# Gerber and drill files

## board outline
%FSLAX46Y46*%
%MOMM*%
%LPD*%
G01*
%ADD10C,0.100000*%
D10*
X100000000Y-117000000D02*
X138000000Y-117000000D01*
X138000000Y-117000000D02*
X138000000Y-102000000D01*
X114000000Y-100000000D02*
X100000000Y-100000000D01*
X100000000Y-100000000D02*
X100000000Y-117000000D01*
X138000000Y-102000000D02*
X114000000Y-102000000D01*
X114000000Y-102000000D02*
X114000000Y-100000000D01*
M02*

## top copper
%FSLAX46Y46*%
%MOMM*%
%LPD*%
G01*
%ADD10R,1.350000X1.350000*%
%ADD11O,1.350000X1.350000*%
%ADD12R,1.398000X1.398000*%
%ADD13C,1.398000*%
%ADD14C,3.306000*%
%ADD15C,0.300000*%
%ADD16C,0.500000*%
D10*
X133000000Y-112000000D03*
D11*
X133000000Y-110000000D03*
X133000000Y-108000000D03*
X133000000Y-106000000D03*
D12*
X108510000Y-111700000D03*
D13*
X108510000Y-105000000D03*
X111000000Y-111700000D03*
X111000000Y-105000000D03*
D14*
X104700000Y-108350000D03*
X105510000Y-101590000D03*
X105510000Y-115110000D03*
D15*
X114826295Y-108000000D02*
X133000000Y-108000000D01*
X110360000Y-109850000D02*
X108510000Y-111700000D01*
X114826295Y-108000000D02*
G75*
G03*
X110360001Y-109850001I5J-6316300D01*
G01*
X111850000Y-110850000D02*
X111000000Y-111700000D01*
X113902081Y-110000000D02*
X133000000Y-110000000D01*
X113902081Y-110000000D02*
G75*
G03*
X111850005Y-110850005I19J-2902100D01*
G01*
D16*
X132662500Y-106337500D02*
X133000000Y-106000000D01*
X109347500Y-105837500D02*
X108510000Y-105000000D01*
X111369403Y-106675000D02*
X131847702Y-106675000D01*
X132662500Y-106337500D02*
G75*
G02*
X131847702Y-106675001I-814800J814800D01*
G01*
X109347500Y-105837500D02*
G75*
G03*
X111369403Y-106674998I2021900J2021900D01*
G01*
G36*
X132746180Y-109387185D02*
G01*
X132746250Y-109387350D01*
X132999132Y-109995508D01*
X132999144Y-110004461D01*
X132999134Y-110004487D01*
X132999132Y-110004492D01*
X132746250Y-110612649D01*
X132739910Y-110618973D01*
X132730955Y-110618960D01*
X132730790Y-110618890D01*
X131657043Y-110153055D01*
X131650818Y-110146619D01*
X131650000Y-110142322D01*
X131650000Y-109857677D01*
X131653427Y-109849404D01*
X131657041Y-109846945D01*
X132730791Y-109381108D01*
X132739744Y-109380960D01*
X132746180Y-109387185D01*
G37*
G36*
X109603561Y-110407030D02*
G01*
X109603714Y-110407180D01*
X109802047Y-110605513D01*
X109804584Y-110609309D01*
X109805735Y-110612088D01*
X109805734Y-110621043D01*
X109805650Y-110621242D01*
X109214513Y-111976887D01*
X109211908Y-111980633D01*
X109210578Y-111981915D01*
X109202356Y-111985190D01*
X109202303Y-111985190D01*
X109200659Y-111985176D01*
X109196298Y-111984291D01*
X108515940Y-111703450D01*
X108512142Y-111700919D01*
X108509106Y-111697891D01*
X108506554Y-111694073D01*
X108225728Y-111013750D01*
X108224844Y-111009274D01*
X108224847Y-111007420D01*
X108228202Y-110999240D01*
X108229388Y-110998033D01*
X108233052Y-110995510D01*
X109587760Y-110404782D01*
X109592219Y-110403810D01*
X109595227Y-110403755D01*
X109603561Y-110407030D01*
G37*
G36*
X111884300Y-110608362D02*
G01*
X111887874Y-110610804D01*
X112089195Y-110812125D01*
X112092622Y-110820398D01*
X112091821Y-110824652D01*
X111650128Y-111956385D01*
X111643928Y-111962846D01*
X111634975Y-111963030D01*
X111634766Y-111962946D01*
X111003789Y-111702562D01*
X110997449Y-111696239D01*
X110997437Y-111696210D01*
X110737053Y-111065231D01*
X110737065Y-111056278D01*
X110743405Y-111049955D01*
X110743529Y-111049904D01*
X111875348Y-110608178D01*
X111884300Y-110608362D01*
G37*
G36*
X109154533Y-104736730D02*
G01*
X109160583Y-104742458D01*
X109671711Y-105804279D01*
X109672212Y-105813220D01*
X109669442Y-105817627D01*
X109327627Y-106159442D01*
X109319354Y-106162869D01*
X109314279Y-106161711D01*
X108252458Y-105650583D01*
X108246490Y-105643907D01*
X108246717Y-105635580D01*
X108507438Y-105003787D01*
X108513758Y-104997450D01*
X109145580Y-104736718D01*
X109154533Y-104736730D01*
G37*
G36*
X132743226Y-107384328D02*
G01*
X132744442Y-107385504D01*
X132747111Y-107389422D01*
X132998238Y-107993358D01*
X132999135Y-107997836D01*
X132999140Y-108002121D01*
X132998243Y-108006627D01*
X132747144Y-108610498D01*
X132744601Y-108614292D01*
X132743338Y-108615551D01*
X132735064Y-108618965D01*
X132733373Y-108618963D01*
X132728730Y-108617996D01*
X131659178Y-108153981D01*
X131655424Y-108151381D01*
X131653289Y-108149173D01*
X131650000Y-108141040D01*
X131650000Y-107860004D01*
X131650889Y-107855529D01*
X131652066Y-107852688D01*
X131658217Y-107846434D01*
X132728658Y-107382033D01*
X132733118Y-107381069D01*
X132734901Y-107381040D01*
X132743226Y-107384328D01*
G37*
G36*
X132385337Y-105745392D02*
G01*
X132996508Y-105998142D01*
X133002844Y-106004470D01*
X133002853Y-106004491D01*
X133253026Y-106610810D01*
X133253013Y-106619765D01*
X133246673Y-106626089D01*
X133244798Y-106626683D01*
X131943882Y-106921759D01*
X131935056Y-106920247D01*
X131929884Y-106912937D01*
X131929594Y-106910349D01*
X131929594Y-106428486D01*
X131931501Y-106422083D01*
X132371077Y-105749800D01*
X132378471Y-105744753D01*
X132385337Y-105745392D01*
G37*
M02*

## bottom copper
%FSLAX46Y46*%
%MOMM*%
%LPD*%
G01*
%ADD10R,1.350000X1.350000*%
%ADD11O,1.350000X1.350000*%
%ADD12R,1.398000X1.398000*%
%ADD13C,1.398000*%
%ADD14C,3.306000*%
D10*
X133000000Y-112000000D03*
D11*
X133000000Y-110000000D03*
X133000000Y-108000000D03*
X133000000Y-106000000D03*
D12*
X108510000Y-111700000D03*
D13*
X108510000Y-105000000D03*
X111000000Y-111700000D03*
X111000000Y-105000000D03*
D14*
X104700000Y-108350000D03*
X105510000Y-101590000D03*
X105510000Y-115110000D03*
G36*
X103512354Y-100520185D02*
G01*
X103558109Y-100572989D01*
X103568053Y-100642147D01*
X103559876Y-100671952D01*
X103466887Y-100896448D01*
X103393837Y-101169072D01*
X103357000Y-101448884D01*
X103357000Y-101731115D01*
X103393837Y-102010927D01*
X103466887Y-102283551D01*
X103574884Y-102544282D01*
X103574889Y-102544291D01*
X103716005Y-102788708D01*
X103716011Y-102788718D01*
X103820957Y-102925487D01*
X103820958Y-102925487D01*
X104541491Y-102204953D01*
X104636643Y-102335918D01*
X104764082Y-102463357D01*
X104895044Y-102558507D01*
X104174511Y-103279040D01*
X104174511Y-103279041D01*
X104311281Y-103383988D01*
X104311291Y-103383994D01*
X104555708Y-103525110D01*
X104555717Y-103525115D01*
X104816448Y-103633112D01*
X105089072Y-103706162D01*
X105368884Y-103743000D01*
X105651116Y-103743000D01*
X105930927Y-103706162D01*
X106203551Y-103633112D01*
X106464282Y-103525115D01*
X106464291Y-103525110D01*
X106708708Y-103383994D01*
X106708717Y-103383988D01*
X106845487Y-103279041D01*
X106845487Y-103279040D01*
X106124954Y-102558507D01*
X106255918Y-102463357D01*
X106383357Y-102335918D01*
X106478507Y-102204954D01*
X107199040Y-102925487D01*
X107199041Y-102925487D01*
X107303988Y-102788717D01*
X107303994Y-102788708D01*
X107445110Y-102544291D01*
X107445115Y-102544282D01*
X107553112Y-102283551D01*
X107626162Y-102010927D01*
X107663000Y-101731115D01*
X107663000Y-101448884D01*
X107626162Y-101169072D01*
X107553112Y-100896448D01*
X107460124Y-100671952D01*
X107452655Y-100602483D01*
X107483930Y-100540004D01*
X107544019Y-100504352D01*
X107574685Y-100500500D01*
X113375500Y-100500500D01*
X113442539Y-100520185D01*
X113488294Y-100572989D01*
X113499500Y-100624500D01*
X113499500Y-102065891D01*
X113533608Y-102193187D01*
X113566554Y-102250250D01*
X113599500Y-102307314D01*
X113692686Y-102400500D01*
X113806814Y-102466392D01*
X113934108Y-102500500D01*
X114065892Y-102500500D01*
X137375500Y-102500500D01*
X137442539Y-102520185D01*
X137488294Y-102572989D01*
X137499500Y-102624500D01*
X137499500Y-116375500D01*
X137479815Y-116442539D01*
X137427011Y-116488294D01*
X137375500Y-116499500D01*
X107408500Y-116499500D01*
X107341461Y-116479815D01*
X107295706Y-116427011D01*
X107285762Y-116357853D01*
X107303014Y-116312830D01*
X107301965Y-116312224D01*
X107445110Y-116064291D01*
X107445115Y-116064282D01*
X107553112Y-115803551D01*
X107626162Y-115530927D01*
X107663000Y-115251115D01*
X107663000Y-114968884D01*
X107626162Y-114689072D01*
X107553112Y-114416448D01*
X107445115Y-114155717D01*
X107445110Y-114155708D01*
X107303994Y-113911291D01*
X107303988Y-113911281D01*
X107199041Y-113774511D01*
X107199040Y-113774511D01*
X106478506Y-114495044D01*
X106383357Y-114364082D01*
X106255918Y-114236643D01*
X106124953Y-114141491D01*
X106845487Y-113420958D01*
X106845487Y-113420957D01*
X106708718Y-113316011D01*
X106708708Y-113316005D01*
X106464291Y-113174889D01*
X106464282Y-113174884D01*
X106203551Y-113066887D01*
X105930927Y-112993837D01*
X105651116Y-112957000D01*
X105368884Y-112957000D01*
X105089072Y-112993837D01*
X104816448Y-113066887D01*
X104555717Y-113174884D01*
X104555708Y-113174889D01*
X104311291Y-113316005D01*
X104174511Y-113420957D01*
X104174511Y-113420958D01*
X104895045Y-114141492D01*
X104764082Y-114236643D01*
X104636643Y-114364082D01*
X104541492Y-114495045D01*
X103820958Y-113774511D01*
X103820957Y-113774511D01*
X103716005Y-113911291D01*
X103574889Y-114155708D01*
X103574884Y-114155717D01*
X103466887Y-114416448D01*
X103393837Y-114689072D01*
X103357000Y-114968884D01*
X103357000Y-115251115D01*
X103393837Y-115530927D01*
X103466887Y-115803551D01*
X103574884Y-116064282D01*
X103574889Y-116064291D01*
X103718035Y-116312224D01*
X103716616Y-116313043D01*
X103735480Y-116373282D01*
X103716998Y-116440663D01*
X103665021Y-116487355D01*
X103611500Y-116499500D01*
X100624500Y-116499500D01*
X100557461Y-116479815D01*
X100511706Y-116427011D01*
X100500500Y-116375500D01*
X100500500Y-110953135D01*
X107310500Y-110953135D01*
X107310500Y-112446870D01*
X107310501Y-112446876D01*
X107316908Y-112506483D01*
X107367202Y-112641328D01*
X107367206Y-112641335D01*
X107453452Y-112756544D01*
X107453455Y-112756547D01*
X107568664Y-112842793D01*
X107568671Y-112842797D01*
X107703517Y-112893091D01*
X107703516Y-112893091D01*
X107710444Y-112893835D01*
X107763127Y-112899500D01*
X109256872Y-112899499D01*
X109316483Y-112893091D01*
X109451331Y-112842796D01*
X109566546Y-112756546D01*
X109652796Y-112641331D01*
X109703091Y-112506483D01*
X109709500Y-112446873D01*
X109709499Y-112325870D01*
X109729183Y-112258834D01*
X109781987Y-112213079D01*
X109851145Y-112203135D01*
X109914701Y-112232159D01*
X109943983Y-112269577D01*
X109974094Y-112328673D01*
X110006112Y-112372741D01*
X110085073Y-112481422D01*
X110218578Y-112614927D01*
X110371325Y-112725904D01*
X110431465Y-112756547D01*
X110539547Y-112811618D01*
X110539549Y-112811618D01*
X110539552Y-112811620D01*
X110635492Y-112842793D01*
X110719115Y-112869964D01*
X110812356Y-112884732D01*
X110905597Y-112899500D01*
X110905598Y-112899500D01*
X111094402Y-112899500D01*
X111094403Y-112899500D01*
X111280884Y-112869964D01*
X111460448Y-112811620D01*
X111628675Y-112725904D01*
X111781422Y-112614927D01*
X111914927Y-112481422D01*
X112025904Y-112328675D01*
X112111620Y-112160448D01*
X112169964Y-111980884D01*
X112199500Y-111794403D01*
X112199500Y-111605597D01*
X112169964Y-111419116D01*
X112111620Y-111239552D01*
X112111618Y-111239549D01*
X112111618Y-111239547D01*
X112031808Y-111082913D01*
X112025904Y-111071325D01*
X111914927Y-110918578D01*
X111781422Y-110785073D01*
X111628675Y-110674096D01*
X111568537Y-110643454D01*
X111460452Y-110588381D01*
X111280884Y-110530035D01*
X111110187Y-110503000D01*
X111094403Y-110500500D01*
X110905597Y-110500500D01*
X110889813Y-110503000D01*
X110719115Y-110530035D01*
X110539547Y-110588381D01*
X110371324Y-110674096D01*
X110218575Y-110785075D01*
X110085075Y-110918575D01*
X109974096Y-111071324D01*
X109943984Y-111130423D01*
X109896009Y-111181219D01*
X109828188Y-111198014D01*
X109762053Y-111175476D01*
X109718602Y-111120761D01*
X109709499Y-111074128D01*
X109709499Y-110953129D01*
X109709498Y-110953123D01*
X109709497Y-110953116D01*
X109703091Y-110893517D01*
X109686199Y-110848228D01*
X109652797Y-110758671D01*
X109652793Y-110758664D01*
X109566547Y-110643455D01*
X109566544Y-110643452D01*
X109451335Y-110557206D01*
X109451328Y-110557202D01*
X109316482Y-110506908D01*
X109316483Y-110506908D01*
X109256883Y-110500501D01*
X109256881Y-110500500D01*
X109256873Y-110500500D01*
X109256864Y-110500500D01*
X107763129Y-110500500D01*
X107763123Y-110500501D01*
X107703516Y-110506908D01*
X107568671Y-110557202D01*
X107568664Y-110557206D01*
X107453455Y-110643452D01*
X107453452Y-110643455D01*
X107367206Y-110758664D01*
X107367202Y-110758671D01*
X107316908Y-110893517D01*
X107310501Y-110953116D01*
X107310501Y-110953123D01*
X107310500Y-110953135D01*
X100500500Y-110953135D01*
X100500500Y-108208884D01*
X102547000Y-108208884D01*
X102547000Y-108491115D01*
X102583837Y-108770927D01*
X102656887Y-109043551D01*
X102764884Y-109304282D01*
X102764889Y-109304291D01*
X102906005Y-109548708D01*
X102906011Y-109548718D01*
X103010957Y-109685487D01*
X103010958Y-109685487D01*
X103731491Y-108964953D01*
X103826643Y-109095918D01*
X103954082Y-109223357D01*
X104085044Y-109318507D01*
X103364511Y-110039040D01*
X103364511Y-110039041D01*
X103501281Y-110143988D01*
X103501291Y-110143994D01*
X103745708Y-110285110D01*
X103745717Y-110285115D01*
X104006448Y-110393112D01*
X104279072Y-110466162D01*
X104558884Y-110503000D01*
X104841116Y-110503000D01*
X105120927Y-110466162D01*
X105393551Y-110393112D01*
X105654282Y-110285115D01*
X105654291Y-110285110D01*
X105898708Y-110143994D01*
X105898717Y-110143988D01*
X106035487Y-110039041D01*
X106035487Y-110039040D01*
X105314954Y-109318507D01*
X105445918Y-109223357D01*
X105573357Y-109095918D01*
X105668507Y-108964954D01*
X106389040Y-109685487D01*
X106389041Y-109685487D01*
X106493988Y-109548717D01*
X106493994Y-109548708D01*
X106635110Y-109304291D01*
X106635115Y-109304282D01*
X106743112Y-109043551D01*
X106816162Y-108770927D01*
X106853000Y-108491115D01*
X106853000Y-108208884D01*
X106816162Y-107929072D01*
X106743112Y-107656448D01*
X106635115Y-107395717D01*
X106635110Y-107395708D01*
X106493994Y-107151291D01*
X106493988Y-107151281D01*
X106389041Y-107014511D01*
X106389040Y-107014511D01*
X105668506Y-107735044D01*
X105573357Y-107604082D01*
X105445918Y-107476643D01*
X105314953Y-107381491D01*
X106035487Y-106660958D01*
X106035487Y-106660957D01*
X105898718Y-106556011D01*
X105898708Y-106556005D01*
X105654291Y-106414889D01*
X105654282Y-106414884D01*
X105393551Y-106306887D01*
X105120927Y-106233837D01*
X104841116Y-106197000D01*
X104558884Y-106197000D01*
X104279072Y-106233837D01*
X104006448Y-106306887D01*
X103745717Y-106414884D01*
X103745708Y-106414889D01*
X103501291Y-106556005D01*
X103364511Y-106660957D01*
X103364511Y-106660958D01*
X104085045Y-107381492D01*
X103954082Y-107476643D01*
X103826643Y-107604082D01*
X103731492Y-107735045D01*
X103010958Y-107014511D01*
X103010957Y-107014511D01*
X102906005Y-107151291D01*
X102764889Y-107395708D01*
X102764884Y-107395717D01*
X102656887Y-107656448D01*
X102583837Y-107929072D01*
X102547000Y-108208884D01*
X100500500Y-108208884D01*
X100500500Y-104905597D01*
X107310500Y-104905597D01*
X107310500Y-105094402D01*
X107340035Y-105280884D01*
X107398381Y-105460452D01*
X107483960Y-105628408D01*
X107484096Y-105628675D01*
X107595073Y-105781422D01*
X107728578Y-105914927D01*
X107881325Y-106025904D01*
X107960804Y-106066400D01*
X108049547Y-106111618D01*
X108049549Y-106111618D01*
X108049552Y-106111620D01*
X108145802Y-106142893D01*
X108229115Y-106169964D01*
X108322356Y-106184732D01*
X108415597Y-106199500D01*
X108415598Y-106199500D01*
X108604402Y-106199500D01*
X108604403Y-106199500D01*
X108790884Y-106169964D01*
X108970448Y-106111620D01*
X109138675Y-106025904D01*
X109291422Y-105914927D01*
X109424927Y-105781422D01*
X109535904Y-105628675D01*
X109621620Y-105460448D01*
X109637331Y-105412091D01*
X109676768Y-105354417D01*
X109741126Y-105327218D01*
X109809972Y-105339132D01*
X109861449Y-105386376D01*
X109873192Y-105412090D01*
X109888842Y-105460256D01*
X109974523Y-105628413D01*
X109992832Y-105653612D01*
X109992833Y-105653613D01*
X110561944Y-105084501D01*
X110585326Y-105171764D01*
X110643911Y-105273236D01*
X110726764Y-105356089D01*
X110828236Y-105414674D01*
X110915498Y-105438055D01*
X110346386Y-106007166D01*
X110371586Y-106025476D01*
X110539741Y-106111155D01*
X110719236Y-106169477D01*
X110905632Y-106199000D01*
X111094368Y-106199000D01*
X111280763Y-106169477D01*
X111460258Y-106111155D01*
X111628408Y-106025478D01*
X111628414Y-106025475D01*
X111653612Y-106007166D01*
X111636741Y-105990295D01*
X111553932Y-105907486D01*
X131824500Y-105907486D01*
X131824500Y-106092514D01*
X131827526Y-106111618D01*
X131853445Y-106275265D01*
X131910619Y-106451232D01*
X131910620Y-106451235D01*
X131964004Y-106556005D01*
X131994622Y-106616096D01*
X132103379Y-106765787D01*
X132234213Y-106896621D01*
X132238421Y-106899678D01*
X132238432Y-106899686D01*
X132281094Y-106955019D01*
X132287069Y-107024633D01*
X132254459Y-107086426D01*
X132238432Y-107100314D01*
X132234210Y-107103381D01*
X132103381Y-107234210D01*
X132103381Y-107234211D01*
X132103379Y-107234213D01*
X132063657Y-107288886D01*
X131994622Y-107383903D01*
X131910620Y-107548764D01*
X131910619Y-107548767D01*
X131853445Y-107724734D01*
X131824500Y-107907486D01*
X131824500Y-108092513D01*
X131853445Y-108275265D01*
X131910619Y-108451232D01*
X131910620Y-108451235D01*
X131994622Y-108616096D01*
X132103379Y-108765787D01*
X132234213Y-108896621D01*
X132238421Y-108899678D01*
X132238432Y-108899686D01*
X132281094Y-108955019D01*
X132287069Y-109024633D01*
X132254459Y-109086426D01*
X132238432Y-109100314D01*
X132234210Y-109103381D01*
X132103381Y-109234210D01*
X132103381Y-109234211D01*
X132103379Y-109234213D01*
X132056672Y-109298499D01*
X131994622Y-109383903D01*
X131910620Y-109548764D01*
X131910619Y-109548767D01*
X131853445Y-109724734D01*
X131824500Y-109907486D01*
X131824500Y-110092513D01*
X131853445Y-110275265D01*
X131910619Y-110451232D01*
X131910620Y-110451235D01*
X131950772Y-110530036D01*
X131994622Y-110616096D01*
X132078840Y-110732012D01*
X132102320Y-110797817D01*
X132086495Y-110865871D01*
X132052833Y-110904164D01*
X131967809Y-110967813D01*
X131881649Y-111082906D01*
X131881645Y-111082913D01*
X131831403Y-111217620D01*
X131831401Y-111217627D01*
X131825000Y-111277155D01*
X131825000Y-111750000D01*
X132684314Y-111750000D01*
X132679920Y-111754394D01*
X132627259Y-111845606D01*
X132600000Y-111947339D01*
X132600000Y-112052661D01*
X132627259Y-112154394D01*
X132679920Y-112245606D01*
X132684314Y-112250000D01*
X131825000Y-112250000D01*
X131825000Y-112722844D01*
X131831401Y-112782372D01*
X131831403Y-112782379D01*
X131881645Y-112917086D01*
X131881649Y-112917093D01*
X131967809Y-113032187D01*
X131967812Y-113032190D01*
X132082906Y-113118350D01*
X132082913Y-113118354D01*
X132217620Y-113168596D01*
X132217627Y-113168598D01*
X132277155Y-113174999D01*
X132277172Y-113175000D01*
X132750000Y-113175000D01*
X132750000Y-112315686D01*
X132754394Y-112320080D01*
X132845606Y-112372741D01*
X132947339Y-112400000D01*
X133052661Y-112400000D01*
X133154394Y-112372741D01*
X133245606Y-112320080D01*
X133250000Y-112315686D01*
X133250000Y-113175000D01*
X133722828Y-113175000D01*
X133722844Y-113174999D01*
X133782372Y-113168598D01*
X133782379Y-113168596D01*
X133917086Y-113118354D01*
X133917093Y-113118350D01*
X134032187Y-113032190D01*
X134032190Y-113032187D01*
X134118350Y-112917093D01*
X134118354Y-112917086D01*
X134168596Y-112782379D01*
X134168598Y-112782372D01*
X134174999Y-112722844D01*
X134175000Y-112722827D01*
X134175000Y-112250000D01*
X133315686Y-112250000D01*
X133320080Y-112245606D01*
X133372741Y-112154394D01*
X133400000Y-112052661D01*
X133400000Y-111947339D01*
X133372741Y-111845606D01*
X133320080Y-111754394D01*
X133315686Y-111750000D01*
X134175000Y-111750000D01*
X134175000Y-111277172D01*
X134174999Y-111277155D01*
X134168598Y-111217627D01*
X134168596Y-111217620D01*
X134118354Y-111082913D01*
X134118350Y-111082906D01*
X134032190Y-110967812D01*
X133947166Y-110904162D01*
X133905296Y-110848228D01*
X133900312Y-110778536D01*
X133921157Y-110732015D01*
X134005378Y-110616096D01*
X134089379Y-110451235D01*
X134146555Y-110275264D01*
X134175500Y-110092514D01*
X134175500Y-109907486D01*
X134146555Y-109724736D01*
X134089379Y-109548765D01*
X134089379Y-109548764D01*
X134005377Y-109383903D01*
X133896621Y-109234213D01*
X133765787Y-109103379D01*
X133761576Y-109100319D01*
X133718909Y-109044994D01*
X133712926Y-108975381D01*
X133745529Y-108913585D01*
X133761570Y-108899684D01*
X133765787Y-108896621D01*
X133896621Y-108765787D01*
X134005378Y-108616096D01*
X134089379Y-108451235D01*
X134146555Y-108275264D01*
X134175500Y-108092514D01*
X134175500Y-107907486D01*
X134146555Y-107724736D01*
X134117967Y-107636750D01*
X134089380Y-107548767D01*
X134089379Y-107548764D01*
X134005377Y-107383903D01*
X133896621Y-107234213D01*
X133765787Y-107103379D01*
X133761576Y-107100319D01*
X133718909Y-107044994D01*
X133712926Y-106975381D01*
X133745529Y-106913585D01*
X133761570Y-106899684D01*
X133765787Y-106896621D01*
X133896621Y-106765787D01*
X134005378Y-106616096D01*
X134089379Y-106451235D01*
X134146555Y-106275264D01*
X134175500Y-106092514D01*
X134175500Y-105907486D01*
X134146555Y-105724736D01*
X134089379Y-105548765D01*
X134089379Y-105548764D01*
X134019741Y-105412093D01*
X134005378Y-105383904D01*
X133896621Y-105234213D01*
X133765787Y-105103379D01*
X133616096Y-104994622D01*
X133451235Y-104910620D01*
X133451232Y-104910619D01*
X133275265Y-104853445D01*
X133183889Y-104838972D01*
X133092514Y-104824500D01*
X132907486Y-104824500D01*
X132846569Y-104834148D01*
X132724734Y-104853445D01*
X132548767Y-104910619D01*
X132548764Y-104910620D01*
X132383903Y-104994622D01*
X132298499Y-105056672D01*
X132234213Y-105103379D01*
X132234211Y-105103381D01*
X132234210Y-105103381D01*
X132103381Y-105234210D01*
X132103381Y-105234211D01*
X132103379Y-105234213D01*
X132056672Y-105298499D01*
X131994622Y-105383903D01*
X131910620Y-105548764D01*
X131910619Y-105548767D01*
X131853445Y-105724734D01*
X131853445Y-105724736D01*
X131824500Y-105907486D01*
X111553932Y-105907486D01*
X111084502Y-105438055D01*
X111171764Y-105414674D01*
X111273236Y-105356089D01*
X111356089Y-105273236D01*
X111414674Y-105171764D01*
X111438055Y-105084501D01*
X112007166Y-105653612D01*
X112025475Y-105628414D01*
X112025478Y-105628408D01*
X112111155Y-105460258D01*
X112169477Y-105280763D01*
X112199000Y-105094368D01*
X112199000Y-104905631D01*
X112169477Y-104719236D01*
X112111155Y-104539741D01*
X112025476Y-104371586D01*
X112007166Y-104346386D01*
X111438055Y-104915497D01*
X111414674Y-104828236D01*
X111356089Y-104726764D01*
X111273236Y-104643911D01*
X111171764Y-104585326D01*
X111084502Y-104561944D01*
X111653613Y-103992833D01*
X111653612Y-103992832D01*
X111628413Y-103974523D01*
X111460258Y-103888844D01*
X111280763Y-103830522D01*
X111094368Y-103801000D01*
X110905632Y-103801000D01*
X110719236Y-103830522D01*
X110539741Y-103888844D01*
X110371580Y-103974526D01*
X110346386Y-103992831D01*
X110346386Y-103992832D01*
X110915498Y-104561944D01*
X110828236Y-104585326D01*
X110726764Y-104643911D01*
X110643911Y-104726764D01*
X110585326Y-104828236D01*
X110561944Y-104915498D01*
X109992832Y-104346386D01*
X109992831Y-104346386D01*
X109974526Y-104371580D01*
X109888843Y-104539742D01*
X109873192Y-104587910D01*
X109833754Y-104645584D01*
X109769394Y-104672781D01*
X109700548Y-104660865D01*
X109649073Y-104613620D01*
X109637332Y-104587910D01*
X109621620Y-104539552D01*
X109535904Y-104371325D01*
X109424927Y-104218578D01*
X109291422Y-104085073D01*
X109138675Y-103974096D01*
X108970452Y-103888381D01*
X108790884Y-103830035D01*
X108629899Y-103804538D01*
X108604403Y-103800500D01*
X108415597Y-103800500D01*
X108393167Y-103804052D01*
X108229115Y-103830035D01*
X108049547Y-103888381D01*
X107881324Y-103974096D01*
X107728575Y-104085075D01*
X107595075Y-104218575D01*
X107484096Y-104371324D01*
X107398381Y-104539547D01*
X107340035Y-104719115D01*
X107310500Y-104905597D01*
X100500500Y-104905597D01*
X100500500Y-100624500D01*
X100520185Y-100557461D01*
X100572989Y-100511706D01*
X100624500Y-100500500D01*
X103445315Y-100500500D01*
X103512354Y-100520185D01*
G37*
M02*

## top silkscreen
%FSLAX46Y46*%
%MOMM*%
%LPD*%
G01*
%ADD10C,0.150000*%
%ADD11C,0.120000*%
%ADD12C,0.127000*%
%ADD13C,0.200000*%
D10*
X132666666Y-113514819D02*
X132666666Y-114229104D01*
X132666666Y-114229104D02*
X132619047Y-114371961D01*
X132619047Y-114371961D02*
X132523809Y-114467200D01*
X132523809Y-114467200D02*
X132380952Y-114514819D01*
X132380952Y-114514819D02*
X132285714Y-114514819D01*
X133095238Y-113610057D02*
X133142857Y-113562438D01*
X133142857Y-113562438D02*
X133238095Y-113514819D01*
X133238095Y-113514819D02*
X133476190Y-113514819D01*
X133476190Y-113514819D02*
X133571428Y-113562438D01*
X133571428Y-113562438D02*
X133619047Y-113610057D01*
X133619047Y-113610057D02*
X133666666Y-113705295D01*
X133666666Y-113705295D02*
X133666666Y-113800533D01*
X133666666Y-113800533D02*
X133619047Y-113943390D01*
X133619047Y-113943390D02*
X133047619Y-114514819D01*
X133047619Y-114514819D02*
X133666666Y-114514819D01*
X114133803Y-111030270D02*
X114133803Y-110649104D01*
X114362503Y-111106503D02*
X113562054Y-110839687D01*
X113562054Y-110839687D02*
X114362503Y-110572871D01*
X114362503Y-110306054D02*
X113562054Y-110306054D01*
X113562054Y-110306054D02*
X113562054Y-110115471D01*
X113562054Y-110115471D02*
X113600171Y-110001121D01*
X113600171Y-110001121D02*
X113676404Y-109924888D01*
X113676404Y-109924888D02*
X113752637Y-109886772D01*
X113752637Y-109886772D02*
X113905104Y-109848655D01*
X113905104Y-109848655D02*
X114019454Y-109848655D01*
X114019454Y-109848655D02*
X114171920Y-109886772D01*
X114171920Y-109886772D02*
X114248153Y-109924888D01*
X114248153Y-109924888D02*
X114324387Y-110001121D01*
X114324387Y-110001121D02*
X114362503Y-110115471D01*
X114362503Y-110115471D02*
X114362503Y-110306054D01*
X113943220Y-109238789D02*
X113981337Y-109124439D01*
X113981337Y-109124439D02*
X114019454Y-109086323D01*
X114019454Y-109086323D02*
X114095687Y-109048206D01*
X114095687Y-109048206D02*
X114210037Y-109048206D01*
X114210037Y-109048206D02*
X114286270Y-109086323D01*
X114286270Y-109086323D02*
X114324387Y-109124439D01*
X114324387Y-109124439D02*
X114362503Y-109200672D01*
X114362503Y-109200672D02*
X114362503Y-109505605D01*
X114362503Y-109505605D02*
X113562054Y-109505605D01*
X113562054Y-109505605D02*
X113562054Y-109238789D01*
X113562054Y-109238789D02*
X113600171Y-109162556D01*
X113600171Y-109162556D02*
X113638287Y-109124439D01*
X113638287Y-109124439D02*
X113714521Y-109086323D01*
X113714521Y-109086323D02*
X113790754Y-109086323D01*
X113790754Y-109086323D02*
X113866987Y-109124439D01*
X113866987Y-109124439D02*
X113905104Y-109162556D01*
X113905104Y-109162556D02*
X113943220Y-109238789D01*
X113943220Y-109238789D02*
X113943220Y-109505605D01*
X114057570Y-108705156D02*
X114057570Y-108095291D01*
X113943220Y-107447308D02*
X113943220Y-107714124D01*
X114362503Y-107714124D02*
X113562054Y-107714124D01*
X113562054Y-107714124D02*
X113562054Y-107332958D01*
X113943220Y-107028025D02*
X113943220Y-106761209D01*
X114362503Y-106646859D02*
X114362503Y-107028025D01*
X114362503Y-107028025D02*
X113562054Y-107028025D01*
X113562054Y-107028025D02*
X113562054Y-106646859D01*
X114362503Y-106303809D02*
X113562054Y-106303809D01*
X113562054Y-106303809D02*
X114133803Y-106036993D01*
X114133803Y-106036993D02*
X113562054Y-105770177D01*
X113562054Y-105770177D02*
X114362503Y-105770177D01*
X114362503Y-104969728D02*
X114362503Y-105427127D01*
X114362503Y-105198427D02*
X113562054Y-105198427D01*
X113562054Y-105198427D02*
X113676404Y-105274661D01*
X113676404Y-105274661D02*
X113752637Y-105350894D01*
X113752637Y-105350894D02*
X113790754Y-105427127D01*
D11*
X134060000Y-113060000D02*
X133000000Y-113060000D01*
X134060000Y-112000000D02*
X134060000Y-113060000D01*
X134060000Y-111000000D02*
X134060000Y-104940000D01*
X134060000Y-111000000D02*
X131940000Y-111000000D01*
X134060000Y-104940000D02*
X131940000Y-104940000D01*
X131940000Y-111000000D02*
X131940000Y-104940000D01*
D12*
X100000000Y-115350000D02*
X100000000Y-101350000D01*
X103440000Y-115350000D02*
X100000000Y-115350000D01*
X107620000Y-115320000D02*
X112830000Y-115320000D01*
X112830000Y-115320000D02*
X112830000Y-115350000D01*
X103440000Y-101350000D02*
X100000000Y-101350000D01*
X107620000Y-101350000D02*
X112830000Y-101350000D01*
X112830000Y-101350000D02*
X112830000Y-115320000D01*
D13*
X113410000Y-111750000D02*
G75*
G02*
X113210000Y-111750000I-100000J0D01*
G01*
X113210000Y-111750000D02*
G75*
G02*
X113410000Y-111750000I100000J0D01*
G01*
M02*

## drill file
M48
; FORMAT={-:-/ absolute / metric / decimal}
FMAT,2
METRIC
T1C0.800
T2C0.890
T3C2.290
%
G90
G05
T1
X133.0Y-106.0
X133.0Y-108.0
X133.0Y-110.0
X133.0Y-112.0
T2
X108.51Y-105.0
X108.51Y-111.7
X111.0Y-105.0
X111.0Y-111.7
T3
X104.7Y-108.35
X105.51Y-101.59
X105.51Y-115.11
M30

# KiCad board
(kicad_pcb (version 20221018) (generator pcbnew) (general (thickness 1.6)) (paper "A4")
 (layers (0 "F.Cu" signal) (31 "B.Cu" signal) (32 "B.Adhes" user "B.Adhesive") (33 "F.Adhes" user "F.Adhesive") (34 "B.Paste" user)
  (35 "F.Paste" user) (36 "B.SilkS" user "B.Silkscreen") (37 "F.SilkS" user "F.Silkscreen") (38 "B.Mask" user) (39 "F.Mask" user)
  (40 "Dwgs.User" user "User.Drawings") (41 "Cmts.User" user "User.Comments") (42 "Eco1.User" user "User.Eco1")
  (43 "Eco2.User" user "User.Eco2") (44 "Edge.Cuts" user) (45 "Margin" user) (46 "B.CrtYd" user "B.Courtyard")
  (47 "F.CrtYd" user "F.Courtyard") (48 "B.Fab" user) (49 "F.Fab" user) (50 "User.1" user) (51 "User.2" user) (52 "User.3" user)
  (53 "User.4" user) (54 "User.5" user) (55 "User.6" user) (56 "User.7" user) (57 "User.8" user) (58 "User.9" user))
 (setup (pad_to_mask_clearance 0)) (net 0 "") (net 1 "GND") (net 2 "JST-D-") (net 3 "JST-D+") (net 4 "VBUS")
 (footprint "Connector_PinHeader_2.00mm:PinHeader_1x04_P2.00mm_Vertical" (layer "F.Cu") (at 133 112 180)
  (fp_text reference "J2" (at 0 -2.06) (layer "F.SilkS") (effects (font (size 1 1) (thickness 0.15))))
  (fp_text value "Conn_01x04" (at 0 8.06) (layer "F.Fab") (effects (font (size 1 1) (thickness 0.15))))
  (fp_line (start -1.06 -1.06) (end 0 -1.06) (stroke (width 0.12) (type solid)) (layer "F.SilkS"))
  (fp_line (start -1.06 0) (end -1.06 -1.06) (stroke (width 0.12) (type solid)) (layer "F.SilkS"))
  (fp_line (start -1.06 1) (end -1.06 7.06) (stroke (width 0.12) (type solid)) (layer "F.SilkS"))
  (fp_line (start -1.06 1) (end 1.06 1) (stroke (width 0.12) (type solid)) (layer "F.SilkS"))
  (fp_line (start -1.06 7.06) (end 1.06 7.06) (stroke (width 0.12) (type solid)) (layer "F.SilkS"))
  (fp_line (start 1.06 1) (end 1.06 7.06) (stroke (width 0.12) (type solid)) (layer "F.SilkS"))
  (pad "1" thru_hole rect (at 0 0 180) (size 1.35 1.35) (drill 0.8) (layers "*.Cu" "*.Mask") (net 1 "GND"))
  (pad "2" thru_hole oval (at 0 2 180) (size 1.35 1.35) (drill 0.8) (layers "*.Cu" "*.Mask") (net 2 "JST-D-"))
  (pad "3" thru_hole oval (at 0 4 180) (size 1.35 1.35) (drill 0.8) (layers "*.Cu" "*.Mask") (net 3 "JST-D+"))
  (pad "4" thru_hole oval (at 0 6 180) (size 1.35 1.35) (drill 0.8) (layers "*.Cu" "*.Mask") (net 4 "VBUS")))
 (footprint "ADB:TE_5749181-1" (layer "F.Cu") (at 108.51 108.35 90)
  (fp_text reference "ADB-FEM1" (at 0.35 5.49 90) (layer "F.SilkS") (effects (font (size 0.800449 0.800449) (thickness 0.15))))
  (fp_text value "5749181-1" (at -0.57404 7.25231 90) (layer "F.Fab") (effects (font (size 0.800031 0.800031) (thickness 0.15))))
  (fp_line (start -7 -8.51) (end 7 -8.51) (stroke (width 0.127) (type solid)) (layer "F.SilkS"))
  (fp_line (start -7 -5.07) (end -7 -8.51) (stroke (width 0.127) (type solid)) (layer "F.SilkS"))
  (fp_line (start -6.97 -0.89) (end -6.97 4.32) (stroke (width 0.127) (type solid)) (layer "F.SilkS"))
  (fp_line (start -6.97 4.32) (end -7 4.32) (stroke (width 0.127) (type solid)) (layer "F.SilkS"))
  (fp_line (start 7 -5.07) (end 7 -8.51) (stroke (width 0.127) (type solid)) (layer "F.SilkS"))
  (fp_line (start 7 -0.89) (end 7 4.32) (stroke (width 0.127) (type solid)) (layer "F.SilkS"))
  (fp_line (start 7 4.32) (end -6.97 4.32) (stroke (width 0.127) (type solid)) (layer "F.SilkS"))
  (fp_circle (center -3.4 4.8) (end -3.3 4.8) (stroke (width 0.2) (type solid)) (fill none) (layer "F.SilkS"))
  (pad "1" thru_hole rect (at -3.35 0 90) (size 1.398 1.398) (drill 0.89) (layers "*.Cu" "*.Mask") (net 3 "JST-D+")
   (solder_mask_margin 0.102))
  (pad "2" thru_hole circle (at 3.35 0 90) (size 1.398 1.398) (drill 0.89) (layers "*.Cu" "*.Mask") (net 4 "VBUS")
   (solder_mask_margin 0.102))
  (pad "3" thru_hole circle (at -3.35 2.49 90) (size 1.398 1.398) (drill 0.89) (layers "*.Cu" "*.Mask") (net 2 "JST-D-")
   (solder_mask_margin 0.102))
  (pad "4" thru_hole circle (at 3.35 2.49 90) (size 1.398 1.398) (drill 0.89) (layers "*.Cu" "*.Mask") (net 1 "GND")
   (solder_mask_margin 0.102))
  (pad "5" thru_hole circle (at 0 -3.81 90) (size 3.306 3.306) (drill 2.29) (layers "*.Cu" "*.Mask") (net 1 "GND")
   (solder_mask_margin 0.102))
  (pad "6" thru_hole circle (at 6.76 -3 90) (size 3.306 3.306) (drill 2.29) (layers "*.Cu" "*.Mask") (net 1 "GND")
   (solder_mask_margin 0.102))
  (pad "7" thru_hole circle (at -6.76 -3 90) (size 3.306 3.306) (drill 2.29) (layers "*.Cu" "*.Mask") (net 1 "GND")
   (solder_mask_margin 0.102)))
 (gr_line (start 100 117) (end 138 117) (stroke (width 0.1) (type default)) (layer "Edge.Cuts"))
 (gr_line (start 138 117) (end 138 102) (stroke (width 0.1) (type default)) (layer "Edge.Cuts"))
 (gr_line (start 114 100) (end 100 100) (stroke (width 0.1) (type default)) (layer "Edge.Cuts"))
 (gr_line (start 100 100) (end 100 117) (stroke (width 0.1) (type default)) (layer "Edge.Cuts"))
 (gr_line (start 138 102) (end 114 102) (stroke (width 0.1) (type default)) (layer "Edge.Cuts"))
 (gr_line (start 114 102) (end 114 100) (stroke (width 0.1) (type default)) (layer "Edge.Cuts"))
 (segment (start 114.826295 108) (end 133 108) (width 0.3) (layer "F.Cu") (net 3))
 (segment (start 110.36 109.85) (end 108.51 111.7) (width 0.3) (layer "F.Cu") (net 3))
 (arc (start 114.826295 108) (mid 112.409153 108.480799) (end 110.36 109.85) (width 0.3) (layer "F.Cu") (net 3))
 (segment (start 111.85 110.85) (end 111 111.7) (width 0.3) (layer "F.Cu") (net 2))
 (segment (start 113.902081 110) (end 133 110) (width 0.3) (layer "F.Cu") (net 2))
 (arc (start 113.902081 110) (mid 112.791502 110.220907) (end 111.85 110.85) (width 0.3) (layer "F.Cu") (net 2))
 (segment (start 132.6625 106.3375) (end 133 106) (width 0.5) (layer "F.Cu") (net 4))
 (segment (start 109.3475 105.8375) (end 108.51 105) (width 0.5) (layer "F.Cu") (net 4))
 (segment (start 111.369403 106.675) (end 131.847702 106.675) (width 0.5) (layer "F.Cu") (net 4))
 (arc (start 132.6625 106.3375) (mid 132.288667 106.587286) (end 131.847702 106.675) (width 0.5) (layer "F.Cu") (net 4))
 (arc (start 109.3475 105.8375) (mid 110.275157 106.45734) (end 111.369403 106.675) (width 0.5) (layer "F.Cu") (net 4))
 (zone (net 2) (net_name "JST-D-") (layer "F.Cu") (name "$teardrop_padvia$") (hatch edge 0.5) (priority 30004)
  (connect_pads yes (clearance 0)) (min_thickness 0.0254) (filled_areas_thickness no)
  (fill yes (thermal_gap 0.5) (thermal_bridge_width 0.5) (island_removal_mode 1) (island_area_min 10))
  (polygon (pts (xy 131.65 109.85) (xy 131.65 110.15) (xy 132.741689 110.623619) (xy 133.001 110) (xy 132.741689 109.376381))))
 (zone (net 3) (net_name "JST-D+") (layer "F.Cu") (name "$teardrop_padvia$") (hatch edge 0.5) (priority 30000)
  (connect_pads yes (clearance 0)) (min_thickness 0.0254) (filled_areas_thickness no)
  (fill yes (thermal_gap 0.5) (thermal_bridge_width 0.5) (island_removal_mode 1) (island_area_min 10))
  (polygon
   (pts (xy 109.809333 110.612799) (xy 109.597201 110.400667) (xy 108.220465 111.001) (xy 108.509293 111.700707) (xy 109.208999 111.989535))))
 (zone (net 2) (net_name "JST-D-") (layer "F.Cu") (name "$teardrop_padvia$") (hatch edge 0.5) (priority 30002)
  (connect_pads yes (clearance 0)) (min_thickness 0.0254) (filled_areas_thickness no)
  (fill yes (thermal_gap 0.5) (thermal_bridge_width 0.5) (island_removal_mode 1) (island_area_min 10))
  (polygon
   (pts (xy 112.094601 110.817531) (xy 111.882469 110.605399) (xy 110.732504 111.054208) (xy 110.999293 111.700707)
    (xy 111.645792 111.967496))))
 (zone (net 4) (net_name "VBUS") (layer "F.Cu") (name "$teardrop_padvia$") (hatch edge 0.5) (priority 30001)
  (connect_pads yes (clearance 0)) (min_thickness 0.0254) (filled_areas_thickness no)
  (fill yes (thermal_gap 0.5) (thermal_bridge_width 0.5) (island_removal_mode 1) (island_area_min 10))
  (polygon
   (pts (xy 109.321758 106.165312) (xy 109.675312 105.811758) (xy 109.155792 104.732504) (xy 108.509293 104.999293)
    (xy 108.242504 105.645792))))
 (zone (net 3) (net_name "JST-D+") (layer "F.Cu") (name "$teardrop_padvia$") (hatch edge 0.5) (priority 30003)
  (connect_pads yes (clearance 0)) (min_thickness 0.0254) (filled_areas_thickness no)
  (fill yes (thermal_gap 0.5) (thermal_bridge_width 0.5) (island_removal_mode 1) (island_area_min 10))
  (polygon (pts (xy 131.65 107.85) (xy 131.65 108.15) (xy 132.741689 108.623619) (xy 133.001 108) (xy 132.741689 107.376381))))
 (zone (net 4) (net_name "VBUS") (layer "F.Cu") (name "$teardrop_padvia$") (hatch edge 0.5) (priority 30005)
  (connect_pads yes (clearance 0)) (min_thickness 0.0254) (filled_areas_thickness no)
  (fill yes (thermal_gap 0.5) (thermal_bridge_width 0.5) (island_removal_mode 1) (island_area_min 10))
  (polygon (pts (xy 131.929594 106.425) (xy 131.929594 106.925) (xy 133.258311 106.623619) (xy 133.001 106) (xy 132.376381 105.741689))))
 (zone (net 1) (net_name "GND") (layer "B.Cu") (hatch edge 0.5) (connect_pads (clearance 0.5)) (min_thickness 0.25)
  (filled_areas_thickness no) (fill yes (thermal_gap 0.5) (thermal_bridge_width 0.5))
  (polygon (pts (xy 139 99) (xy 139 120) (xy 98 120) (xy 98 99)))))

